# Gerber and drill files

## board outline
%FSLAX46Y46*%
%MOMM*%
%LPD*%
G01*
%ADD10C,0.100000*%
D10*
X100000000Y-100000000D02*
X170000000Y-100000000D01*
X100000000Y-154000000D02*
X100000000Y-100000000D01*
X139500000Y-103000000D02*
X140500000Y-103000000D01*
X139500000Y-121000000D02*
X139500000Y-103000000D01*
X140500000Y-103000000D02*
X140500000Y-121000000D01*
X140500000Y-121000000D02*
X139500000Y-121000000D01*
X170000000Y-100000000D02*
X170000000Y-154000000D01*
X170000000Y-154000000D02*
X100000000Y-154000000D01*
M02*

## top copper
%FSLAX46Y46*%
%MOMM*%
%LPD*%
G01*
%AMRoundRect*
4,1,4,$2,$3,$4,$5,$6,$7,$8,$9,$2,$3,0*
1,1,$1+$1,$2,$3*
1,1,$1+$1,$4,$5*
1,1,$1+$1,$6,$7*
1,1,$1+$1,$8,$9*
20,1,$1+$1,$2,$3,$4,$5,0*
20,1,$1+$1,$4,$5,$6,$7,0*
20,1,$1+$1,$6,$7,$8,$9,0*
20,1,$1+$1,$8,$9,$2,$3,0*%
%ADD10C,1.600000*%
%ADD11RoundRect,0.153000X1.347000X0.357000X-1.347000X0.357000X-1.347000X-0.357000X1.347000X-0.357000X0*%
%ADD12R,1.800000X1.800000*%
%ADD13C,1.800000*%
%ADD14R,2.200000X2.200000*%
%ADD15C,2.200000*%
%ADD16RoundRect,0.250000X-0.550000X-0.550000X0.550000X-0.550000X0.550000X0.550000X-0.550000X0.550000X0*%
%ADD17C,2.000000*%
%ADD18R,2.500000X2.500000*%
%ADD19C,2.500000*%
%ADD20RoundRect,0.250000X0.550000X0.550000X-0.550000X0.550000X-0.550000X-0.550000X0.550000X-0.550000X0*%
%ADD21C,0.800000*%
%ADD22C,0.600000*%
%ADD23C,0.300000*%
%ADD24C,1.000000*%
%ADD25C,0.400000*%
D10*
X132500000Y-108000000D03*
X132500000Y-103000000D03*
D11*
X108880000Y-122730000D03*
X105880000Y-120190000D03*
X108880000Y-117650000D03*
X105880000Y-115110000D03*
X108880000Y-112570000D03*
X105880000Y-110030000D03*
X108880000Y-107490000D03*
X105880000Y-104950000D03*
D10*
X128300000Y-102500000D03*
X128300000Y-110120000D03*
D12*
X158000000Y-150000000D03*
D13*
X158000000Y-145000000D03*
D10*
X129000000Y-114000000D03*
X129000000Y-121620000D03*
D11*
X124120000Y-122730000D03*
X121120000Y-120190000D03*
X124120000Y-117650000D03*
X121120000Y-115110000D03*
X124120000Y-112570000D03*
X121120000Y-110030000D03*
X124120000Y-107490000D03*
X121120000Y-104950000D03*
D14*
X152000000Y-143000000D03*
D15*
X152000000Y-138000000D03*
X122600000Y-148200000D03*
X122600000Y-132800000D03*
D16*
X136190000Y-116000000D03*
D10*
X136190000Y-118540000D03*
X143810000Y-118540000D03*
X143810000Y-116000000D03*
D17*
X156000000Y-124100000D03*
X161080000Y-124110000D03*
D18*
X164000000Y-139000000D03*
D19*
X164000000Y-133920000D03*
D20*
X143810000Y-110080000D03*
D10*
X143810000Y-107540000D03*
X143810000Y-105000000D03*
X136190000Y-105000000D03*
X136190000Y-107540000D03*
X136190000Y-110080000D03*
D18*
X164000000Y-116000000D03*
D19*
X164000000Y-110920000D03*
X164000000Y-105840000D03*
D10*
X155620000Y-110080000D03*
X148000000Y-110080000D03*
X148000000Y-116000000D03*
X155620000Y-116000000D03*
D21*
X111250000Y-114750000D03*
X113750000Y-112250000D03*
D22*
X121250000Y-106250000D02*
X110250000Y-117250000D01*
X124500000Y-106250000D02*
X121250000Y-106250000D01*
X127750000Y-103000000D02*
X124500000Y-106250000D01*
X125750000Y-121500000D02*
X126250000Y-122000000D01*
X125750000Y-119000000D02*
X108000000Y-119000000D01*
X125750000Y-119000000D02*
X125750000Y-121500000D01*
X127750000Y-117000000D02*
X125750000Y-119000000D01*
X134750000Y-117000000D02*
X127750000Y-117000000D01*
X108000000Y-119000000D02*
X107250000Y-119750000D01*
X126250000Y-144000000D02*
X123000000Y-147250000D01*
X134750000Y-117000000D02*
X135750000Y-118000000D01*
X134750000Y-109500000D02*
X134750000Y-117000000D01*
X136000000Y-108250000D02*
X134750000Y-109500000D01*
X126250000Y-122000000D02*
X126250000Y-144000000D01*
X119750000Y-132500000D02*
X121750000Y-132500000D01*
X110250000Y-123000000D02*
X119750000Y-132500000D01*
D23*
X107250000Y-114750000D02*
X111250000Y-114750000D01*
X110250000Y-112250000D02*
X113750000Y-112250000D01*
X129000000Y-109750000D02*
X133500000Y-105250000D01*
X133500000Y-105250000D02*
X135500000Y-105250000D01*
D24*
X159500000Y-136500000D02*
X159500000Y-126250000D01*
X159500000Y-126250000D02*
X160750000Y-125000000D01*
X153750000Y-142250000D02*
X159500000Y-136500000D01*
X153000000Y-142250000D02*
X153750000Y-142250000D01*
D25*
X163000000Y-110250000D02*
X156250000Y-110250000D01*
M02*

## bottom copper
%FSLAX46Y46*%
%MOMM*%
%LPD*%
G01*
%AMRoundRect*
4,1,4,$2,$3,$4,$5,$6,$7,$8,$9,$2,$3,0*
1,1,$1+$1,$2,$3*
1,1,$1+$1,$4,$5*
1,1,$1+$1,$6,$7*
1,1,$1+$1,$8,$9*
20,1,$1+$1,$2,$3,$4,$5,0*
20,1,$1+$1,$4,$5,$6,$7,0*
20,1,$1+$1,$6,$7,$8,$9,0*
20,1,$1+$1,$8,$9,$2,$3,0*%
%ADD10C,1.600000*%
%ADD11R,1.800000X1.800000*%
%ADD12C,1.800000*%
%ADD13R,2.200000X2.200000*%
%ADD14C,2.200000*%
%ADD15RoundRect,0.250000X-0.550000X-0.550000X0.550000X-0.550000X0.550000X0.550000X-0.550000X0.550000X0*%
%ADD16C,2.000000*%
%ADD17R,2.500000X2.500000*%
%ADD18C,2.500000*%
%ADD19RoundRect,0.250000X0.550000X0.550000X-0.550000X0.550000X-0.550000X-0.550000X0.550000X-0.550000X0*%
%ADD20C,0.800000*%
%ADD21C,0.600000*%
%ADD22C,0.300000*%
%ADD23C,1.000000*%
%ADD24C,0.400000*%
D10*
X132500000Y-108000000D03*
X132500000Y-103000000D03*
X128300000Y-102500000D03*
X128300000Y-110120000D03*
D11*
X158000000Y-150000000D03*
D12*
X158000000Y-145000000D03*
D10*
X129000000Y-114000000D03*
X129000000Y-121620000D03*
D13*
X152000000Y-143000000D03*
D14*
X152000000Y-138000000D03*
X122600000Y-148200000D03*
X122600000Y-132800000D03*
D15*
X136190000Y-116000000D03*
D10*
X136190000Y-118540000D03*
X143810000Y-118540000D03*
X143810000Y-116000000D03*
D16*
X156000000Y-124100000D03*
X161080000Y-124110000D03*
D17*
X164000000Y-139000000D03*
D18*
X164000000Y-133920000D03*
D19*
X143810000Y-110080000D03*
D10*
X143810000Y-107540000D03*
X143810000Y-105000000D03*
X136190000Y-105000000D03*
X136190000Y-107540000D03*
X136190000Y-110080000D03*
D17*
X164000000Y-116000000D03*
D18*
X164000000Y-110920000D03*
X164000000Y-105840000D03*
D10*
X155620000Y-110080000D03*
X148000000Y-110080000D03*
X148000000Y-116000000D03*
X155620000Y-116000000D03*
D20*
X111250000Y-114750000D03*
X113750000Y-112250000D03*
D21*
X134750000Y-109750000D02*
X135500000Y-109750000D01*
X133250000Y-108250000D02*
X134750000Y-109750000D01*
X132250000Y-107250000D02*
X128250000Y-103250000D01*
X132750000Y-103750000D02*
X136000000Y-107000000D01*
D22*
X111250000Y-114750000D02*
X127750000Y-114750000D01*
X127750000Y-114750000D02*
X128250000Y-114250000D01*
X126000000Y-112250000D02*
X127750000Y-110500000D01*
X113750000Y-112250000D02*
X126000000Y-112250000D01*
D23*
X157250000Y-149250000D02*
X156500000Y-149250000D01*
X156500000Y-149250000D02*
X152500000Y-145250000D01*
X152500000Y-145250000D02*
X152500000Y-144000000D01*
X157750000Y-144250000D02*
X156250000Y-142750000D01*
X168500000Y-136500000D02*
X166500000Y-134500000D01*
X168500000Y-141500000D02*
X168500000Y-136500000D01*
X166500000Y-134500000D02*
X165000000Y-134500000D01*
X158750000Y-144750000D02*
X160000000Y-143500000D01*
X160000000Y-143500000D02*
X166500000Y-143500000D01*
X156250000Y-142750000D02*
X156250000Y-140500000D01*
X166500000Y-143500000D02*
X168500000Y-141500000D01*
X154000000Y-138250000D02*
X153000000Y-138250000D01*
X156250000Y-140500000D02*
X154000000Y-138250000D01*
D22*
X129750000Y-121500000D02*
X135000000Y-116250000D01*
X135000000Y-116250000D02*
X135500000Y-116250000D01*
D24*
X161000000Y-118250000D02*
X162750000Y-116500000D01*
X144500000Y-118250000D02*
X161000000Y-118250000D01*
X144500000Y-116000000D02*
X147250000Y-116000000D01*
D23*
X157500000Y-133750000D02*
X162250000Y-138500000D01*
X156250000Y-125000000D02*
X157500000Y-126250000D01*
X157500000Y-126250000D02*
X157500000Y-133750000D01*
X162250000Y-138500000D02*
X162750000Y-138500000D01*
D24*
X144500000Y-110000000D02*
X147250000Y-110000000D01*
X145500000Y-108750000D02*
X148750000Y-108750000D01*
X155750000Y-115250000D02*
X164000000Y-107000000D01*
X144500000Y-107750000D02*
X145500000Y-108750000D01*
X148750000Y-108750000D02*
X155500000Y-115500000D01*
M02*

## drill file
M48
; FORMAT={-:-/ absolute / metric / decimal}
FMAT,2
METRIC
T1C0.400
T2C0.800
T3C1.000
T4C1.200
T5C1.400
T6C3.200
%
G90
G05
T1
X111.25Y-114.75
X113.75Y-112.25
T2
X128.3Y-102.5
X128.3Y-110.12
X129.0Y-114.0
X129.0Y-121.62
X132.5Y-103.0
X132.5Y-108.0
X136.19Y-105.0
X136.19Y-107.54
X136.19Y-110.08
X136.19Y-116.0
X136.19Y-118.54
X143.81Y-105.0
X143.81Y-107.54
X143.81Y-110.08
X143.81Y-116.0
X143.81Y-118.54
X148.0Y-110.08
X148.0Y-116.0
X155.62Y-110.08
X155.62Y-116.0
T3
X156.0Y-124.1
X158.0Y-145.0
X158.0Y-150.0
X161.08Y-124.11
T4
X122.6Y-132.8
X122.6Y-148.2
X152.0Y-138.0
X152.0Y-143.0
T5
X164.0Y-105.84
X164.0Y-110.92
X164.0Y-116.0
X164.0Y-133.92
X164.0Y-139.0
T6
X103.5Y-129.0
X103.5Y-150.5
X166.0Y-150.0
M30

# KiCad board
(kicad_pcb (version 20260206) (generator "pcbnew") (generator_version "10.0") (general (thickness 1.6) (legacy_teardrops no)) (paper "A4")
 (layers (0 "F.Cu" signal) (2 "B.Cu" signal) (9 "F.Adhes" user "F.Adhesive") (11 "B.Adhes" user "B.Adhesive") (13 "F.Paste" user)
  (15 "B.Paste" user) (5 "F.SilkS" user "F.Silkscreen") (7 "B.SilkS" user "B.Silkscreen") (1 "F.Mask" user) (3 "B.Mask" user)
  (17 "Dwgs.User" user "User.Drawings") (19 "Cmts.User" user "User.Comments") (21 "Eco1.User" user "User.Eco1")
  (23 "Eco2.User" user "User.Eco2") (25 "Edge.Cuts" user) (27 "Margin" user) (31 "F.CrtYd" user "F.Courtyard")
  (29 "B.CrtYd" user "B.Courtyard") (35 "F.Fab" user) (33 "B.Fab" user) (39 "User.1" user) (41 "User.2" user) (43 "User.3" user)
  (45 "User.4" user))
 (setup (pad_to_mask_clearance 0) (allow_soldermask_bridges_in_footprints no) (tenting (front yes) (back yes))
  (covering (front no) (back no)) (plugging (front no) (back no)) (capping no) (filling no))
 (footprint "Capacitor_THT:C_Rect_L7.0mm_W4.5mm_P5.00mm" (layer "F.Cu") (at 132.5 108 90)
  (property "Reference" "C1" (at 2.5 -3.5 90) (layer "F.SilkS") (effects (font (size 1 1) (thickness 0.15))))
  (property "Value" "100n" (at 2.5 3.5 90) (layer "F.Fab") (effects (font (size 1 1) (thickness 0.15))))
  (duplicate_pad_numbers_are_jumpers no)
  (pad "1" thru_hole circle (at 0 0 90) (size 1.6 1.6) (drill 0.8) (layers "*.Cu" "*.Mask") (remove_unused_layers no) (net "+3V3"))
  (pad "2" thru_hole circle (at 5 0 90) (size 1.6 1.6) (drill 0.8) (layers "*.Cu" "*.Mask") (remove_unused_layers no) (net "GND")))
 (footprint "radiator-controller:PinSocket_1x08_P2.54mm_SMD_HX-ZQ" (layer "F.Cu") (at 107.38 113.84 180)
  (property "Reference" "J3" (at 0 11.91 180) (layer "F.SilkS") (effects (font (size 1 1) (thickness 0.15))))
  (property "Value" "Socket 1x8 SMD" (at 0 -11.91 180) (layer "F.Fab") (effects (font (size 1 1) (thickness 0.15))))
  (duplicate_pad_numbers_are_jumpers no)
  (pad "1" smd roundrect (at -1.5 -8.89 180) (size 3 1.02) (layers "F.Cu" "F.Mask" "F.Paste") (roundrect_rratio 0.15) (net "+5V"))
  (pad "2" smd roundrect (at 1.5 -6.35 180) (size 3 1.02) (layers "F.Cu" "F.Mask" "F.Paste") (roundrect_rratio 0.15) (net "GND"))
  (pad "3" smd roundrect (at -1.5 -3.81 180) (size 3 1.02) (layers "F.Cu" "F.Mask" "F.Paste") (roundrect_rratio 0.15) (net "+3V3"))
  (pad "4" smd roundrect (at 1.5 -1.27 180) (size 3 1.02) (layers "F.Cu" "F.Mask" "F.Paste") (roundrect_rratio 0.15) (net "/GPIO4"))
  (pad "5" smd roundrect (at -1.5 1.27 180) (size 3 1.02) (layers "F.Cu" "F.Mask" "F.Paste") (roundrect_rratio 0.15) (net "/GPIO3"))
  (pad "6" smd roundrect (at 1.5 3.81 180) (size 3 1.02) (layers "F.Cu" "F.Mask" "F.Paste") (roundrect_rratio 0.15) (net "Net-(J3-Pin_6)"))
  (pad "7" smd roundrect (at -1.5 6.35 180) (size 3 1.02) (layers "F.Cu" "F.Mask" "F.Paste") (roundrect_rratio 0.15) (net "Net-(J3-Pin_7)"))
  (pad "8" smd roundrect (at 1.5 8.89 180) (size 3 1.02) (layers "F.Cu" "F.Mask" "F.Paste") (roundrect_rratio 0.15) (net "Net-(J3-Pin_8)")))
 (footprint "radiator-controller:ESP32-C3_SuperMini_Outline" (layer "F.Cu") (at 115 113 180)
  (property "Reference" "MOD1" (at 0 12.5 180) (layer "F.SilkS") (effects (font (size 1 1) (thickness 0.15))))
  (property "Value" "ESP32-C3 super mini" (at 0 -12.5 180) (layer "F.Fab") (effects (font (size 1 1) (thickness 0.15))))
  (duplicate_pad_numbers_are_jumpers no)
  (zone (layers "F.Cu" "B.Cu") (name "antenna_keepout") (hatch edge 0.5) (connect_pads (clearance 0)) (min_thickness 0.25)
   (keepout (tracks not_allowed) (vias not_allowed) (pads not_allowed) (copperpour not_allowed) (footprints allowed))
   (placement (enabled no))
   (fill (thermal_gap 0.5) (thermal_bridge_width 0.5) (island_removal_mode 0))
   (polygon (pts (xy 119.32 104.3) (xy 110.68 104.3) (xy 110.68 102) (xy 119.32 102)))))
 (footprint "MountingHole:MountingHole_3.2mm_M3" (layer "F.Cu") (at 166 150)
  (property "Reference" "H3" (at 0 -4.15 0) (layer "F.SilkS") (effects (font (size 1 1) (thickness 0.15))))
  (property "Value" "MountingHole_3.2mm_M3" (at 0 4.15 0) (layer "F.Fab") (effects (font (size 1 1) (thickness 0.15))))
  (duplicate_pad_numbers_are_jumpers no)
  (pad "" np_thru_hole circle (at 0 0) (size 3.2 3.2) (drill 3.2) (layers "*.Cu" "*.Mask")))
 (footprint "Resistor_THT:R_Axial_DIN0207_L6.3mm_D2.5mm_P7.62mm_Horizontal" (layer "F.Cu") (at 128.3 102.5 -90)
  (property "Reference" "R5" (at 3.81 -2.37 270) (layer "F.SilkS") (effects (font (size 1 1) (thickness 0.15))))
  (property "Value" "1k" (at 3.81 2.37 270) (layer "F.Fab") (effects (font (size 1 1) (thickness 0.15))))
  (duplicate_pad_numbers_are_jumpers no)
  (pad "1" thru_hole circle (at 0 0 270) (size 1.6 1.6) (drill 0.8) (layers "*.Cu" "*.Mask") (remove_unused_layers no) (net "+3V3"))
  (pad "2" thru_hole circle (at 7.62 0 270) (size 1.6 1.6) (drill 0.8) (layers "*.Cu" "*.Mask") (remove_unused_layers no) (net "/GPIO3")))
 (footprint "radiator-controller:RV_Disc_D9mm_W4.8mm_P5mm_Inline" (layer "F.Cu") (at 158 150 90)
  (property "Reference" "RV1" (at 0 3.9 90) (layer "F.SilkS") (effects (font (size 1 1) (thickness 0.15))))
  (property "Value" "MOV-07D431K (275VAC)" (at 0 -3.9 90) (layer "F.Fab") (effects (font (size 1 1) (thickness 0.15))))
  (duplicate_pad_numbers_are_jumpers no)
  (pad "1" thru_hole rect (at 0 0 90) (size 1.8 1.8) (drill 1) (layers "*.Cu" "*.Mask") (remove_unused_layers no) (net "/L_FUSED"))
  (pad "2" thru_hole circle (at 5 0 90) (size 1.8 1.8) (drill 1) (layers "*.Cu" "*.Mask") (remove_unused_layers no) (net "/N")))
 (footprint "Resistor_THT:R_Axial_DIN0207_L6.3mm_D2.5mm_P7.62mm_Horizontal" (layer "F.Cu") (at 129 114 -90)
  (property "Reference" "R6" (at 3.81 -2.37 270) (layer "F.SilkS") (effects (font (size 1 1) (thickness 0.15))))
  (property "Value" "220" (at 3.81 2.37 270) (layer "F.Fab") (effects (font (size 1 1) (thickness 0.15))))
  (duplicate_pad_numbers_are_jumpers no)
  (pad "1" thru_hole circle (at 0 0 270) (size 1.6 1.6) (drill 0.8) (layers "*.Cu" "*.Mask") (remove_unused_layers no) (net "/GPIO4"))
  (pad "2" thru_hole circle (at 7.62 0 270) (size 1.6 1.6) (drill 0.8) (layers "*.Cu" "*.Mask") (remove_unused_layers no)
   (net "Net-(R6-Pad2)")))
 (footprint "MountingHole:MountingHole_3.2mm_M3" (layer "F.Cu") (at 103.5 129)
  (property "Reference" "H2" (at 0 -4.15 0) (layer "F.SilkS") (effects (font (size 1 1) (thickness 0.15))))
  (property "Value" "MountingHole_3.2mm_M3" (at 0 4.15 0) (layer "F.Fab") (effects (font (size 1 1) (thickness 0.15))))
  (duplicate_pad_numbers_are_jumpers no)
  (pad "" np_thru_hole circle (at 0 0) (size 3.2 3.2) (drill 3.2) (layers "*.Cu" "*.Mask")))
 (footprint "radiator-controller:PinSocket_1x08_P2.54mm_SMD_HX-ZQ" (layer "F.Cu") (at 122.62 113.84 180)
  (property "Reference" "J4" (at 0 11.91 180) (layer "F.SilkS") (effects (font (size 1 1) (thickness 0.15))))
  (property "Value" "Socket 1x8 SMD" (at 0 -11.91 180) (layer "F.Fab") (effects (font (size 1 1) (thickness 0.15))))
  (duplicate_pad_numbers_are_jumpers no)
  (pad "1" smd roundrect (at -1.5 -8.89 180) (size 3 1.02) (layers "F.Cu" "F.Mask" "F.Paste") (roundrect_rratio 0.15) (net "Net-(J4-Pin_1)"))
  (pad "2" smd roundrect (at 1.5 -6.35 180) (size 3 1.02) (layers "F.Cu" "F.Mask" "F.Paste") (roundrect_rratio 0.15) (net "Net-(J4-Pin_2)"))
  (pad "3" smd roundrect (at -1.5 -3.81 180) (size 3 1.02) (layers "F.Cu" "F.Mask" "F.Paste") (roundrect_rratio 0.15) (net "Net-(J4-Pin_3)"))
  (pad "4" smd roundrect (at 1.5 -1.27 180) (size 3 1.02) (layers "F.Cu" "F.Mask" "F.Paste") (roundrect_rratio 0.15) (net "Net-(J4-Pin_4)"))
  (pad "5" smd roundrect (at -1.5 1.27 180) (size 3 1.02) (layers "F.Cu" "F.Mask" "F.Paste") (roundrect_rratio 0.15) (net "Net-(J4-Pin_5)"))
  (pad "6" smd roundrect (at 1.5 3.81 180) (size 3 1.02) (layers "F.Cu" "F.Mask" "F.Paste") (roundrect_rratio 0.15) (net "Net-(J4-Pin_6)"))
  (pad "7" smd roundrect (at -1.5 6.35 180) (size 3 1.02) (layers "F.Cu" "F.Mask" "F.Paste") (roundrect_rratio 0.15) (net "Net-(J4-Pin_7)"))
  (pad "8" smd roundrect (at 1.5 8.89 180) (size 3 1.02) (layers "F.Cu" "F.Mask" "F.Paste") (roundrect_rratio 0.15) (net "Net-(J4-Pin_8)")))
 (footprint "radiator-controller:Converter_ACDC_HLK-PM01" (layer "F.Cu") (at 152 143 180)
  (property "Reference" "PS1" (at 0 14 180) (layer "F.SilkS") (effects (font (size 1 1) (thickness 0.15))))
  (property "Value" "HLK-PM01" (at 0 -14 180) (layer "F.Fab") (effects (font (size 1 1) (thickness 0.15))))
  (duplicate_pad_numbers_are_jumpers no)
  (pad "1" thru_hole rect (at 0 0 180) (size 2.2 2.2) (drill 1.2) (layers "*.Cu" "*.Mask") (remove_unused_layers no) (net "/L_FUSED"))
  (pad "2" thru_hole circle (at 0 5 180) (size 2.2 2.2) (drill 1.2) (layers "*.Cu" "*.Mask") (remove_unused_layers no) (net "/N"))
  (pad "3" thru_hole circle (at 29.4 -5.2 180) (size 2.2 2.2) (drill 1.2) (layers "*.Cu" "*.Mask") (remove_unused_layers no) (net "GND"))
  (pad "4" thru_hole circle (at 29.4 10.2 180) (size 2.2 2.2) (drill 1.2) (layers "*.Cu" "*.Mask") (remove_unused_layers no) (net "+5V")))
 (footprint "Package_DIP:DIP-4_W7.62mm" (layer "F.Cu") (at 136.19 116)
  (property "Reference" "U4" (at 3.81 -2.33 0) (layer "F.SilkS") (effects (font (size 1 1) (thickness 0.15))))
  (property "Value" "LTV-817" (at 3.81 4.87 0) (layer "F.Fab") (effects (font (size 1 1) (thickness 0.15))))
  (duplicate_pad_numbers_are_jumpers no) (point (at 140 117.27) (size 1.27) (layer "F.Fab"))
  (pad "1" thru_hole roundrect (at 0 0) (size 1.6 1.6) (drill 0.8) (layers "*.Cu" "*.Mask") (remove_unused_layers no)
   (roundrect_rratio 0.15625) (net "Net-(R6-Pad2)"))
  (pad "2" thru_hole circle (at 0 2.54) (size 1.6 1.6) (drill 0.8) (layers "*.Cu" "*.Mask") (remove_unused_layers no) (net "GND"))
  (pad "3" thru_hole circle (at 7.62 2.54) (size 1.6 1.6) (drill 0.8) (layers "*.Cu" "*.Mask") (remove_unused_layers no) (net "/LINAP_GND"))
  (pad "4" thru_hole circle (at 7.62 0) (size 1.6 1.6) (drill 0.8) (layers "*.Cu" "*.Mask") (remove_unused_layers no) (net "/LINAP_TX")))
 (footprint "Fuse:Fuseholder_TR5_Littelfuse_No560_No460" (layer "F.Cu") (at 156 124.1)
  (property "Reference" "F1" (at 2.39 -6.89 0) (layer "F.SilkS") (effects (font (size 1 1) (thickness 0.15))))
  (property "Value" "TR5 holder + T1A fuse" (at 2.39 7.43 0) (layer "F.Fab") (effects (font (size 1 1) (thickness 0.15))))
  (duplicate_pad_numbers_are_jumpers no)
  (pad "1" thru_hole circle (at 0 0) (size 2 2) (drill 1) (layers "*.Cu" "*.Mask") (remove_unused_layers no) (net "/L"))
  (pad "2" thru_hole circle (at 5.08 0.01) (size 2 2) (drill 1) (layers "*.Cu" "*.Mask") (remove_unused_layers no) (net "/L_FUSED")))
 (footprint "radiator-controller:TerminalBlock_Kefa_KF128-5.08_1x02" (layer "F.Cu") (at 164 139 90)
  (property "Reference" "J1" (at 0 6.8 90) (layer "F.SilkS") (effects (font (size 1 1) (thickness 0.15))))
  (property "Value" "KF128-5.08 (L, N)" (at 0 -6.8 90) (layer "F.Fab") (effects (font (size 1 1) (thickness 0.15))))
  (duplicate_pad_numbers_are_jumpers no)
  (pad "1" thru_hole rect (at 0 0 90) (size 2.5 2.5) (drill 1.4) (layers "*.Cu" "*.Mask") (remove_unused_layers no) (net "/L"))
  (pad "2" thru_hole circle (at 5.08 0 90) (size 2.5 2.5) (drill 1.4) (layers "*.Cu" "*.Mask") (remove_unused_layers no) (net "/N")))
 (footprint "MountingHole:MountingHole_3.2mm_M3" (layer "F.Cu") (at 103.5 150.5)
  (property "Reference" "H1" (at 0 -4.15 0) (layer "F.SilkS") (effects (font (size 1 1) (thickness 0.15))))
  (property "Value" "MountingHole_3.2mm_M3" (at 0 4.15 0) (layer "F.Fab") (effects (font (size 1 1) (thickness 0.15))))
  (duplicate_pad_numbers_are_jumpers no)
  (pad "" np_thru_hole circle (at 0 0) (size 3.2 3.2) (drill 3.2) (layers "*.Cu" "*.Mask")))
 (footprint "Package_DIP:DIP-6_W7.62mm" (layer "F.Cu") (at 143.81 110.08 180)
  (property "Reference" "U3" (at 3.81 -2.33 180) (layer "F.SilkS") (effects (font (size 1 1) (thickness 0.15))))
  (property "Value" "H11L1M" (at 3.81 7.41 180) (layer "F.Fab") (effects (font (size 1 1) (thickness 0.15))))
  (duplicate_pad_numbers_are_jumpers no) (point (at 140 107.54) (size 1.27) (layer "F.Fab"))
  (pad "1" thru_hole roundrect (at 0 0 180) (size 1.6 1.6) (drill 0.8) (layers "*.Cu" "*.Mask") (remove_unused_layers no)
   (roundrect_rratio 0.15625) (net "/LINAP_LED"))
  (pad "2" thru_hole circle (at 0 2.54 180) (size 1.6 1.6) (drill 0.8) (layers "*.Cu" "*.Mask") (remove_unused_layers no)
   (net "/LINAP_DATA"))
  (pad "3" thru_hole circle (at 0 5.08 180) (size 1.6 1.6) (drill 0.8) (layers "*.Cu" "*.Mask") (remove_unused_layers no)
   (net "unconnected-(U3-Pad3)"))
  (pad "4" thru_hole circle (at 7.62 5.08 180) (size 1.6 1.6) (drill 0.8) (layers "*.Cu" "*.Mask") (remove_unused_layers no) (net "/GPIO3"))
  (pad "5" thru_hole circle (at 7.62 2.54 180) (size 1.6 1.6) (drill 0.8) (layers "*.Cu" "*.Mask") (remove_unused_layers no) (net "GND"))
  (pad "6" thru_hole circle (at 7.62 0 180) (size 1.6 1.6) (drill 0.8) (layers "*.Cu" "*.Mask") (remove_unused_layers no) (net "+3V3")))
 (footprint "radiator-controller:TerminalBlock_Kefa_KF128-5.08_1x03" (layer "F.Cu") (at 164 116 90)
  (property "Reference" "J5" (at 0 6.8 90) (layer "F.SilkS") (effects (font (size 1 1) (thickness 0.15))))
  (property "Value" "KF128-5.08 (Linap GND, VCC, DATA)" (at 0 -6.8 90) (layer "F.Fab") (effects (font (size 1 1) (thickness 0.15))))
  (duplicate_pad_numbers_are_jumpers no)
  (pad "1" thru_hole rect (at 0 0 90) (size 2.5 2.5) (drill 1.4) (layers "*.Cu" "*.Mask") (remove_unused_layers no) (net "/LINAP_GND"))
  (pad "2" thru_hole circle (at 5.08 0 90) (size 2.5 2.5) (drill 1.4) (layers "*.Cu" "*.Mask") (remove_unused_layers no) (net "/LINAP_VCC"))
  (pad "3" thru_hole circle (at 10.16 0 90) (size 2.5 2.5) (drill 1.4) (layers "*.Cu" "*.Mask") (remove_unused_layers no)
   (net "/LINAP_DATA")))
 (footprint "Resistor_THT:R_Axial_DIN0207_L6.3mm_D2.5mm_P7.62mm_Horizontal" (layer "F.Cu") (at 155.62 110.08 180)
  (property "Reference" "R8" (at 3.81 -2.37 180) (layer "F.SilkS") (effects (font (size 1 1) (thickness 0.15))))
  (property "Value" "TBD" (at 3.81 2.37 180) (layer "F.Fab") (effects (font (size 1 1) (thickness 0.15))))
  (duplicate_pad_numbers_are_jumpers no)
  (pad "1" thru_hole circle (at 0 0 180) (size 1.6 1.6) (drill 0.8) (layers "*.Cu" "*.Mask") (remove_unused_layers no) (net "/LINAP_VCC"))
  (pad "2" thru_hole circle (at 7.62 0 180) (size 1.6 1.6) (drill 0.8) (layers "*.Cu" "*.Mask") (remove_unused_layers no) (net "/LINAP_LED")))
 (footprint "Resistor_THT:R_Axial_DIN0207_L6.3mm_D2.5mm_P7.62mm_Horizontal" (layer "F.Cu") (at 148 116)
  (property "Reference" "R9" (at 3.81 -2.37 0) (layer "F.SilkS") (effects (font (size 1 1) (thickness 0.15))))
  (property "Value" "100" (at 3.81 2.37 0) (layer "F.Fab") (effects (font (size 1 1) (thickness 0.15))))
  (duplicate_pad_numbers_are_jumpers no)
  (pad "1" thru_hole circle (at 0 0) (size 1.6 1.6) (drill 0.8) (layers "*.Cu" "*.Mask") (remove_unused_layers no) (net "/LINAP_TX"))
  (pad "2" thru_hole circle (at 7.62 0) (size 1.6 1.6) (drill 0.8) (layers "*.Cu" "*.Mask") (remove_unused_layers no) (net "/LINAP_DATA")))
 (gr_line (start 100 100) (end 170 100) (stroke (width 0.1) (type default)) (layer "Edge.Cuts"))
 (gr_line (start 100 154) (end 100 100) (stroke (width 0.1) (type default)) (layer "Edge.Cuts"))
 (gr_line (start 139.5 103) (end 140.5 103) (stroke (width 0.1) (type default)) (layer "Edge.Cuts"))
 (gr_line (start 139.5 121) (end 139.5 103) (stroke (width 0.1) (type default)) (layer "Edge.Cuts"))
 (gr_line (start 140.5 103) (end 140.5 121) (stroke (width 0.1) (type default)) (layer "Edge.Cuts"))
 (gr_line (start 140.5 121) (end 139.5 121) (stroke (width 0.1) (type default)) (layer "Edge.Cuts"))
 (gr_line (start 170 100) (end 170 154) (stroke (width 0.1) (type default)) (layer "Edge.Cuts"))
 (gr_line (start 170 154) (end 100 154) (stroke (width 0.1) (type default)) (layer "Edge.Cuts"))
 (segment (start 121.25 106.25) (end 110.25 117.25) (width 0.6) (layer "F.Cu") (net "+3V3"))
 (segment (start 124.5 106.25) (end 121.25 106.25) (width 0.6) (layer "F.Cu") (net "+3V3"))
 (segment (start 127.75 103) (end 124.5 106.25) (width 0.6) (layer "F.Cu") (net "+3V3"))
 (segment (start 134.75 109.75) (end 135.5 109.75) (width 0.6) (layer "B.Cu") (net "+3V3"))
 (segment (start 133.25 108.25) (end 134.75 109.75) (width 0.6) (layer "B.Cu") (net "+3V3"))
 (segment (start 132.25 107.25) (end 128.25 103.25) (width 0.6) (layer "B.Cu") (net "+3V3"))
 (segment (start 125.75 121.5) (end 126.25 122) (width 0.6) (layer "F.Cu") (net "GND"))
 (segment (start 125.75 119) (end 108 119) (width 0.6) (layer "F.Cu") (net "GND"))
 (segment (start 125.75 119) (end 125.75 121.5) (width 0.6) (layer "F.Cu") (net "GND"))
 (segment (start 127.75 117) (end 125.75 119) (width 0.6) (layer "F.Cu") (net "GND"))
 (segment (start 134.75 117) (end 127.75 117) (width 0.6) (layer "F.Cu") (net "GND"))
 (segment (start 108 119) (end 107.25 119.75) (width 0.6) (layer "F.Cu") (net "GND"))
 (segment (start 126.25 144) (end 123 147.25) (width 0.6) (layer "F.Cu") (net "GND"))
 (segment (start 134.75 117) (end 135.75 118) (width 0.6) (layer "F.Cu") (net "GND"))
 (segment (start 134.75 109.5) (end 134.75 117) (width 0.6) (layer "F.Cu") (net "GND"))
 (segment (start 136 108.25) (end 134.75 109.5) (width 0.6) (layer "F.Cu") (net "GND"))
 (segment (start 126.25 122) (end 126.25 144) (width 0.6) (layer "F.Cu") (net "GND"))
 (segment (start 132.75 103.75) (end 136 107) (width 0.6) (layer "B.Cu") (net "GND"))
 (segment (start 119.75 132.5) (end 121.75 132.5) (width 0.6) (layer "F.Cu") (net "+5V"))
 (segment (start 110.25 123) (end 119.75 132.5) (width 0.6) (layer "F.Cu") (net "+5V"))
 (segment (start 107.25 114.75) (end 111.25 114.75) (width 0.3) (layer "F.Cu") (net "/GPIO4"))
 (via (at 111.25 114.75) (size 0.8) (drill 0.4) (layers "F.Cu" "B.Cu") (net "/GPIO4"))
 (segment (start 111.25 114.75) (end 127.75 114.75) (width 0.3) (layer "B.Cu") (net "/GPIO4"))
 (segment (start 127.75 114.75) (end 128.25 114.25) (width 0.3) (layer "B.Cu") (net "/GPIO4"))
 (segment (start 110.25 112.25) (end 113.75 112.25) (width 0.3) (layer "F.Cu") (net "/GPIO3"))
 (segment (start 129 109.75) (end 133.5 105.25) (width 0.3) (layer "F.Cu") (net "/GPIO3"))
 (segment (start 133.5 105.25) (end 135.5 105.25) (width 0.3) (layer "F.Cu") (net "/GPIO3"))
 (via (at 113.75 112.25) (size 0.8) (drill 0.4) (layers "F.Cu" "B.Cu") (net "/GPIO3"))
 (segment (start 126 112.25) (end 127.75 110.5) (width 0.3) (layer "B.Cu") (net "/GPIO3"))
 (segment (start 113.75 112.25) (end 126 112.25) (width 0.3) (layer "B.Cu") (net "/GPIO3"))
 (segment (start 159.5 136.5) (end 159.5 126.25) (width 1) (layer "F.Cu") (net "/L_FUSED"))
 (segment (start 159.5 126.25) (end 160.75 125) (width 1) (layer "F.Cu") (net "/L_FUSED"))
 (segment (start 153.75 142.25) (end 159.5 136.5) (width 1) (layer "F.Cu") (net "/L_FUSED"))
 (segment (start 153 142.25) (end 153.75 142.25) (width 1) (layer "F.Cu") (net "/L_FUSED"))
 (segment (start 157.25 149.25) (end 156.5 149.25) (width 1) (layer "B.Cu") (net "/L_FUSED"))
 (segment (start 156.5 149.25) (end 152.5 145.25) (width 1) (layer "B.Cu") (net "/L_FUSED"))
 (segment (start 152.5 145.25) (end 152.5 144) (width 1) (layer "B.Cu") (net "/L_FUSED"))
 (segment (start 157.75 144.25) (end 156.25 142.75) (width 1) (layer "B.Cu") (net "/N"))
 (segment (start 168.5 136.5) (end 166.5 134.5) (width 1) (layer "B.Cu") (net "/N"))
 (segment (start 168.5 141.5) (end 168.5 136.5) (width 1) (layer "B.Cu") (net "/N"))
 (segment (start 166.5 134.5) (end 165 134.5) (width 1) (layer "B.Cu") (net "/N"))
 (segment (start 158.75 144.75) (end 160 143.5) (width 1) (layer "B.Cu") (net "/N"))
 (segment (start 160 143.5) (end 166.5 143.5) (width 1) (layer "B.Cu") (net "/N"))
 (segment (start 156.25 142.75) (end 156.25 140.5) (width 1) (layer "B.Cu") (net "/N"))
 (segment (start 166.5 143.5) (end 168.5 141.5) (width 1) (layer "B.Cu") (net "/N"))
 (segment (start 154 138.25) (end 153 138.25) (width 1) (layer "B.Cu") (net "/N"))
 (segment (start 156.25 140.5) (end 154 138.25) (width 1) (layer "B.Cu") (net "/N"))
 (segment (start 129.75 121.5) (end 135 116.25) (width 0.3) (layer "B.Cu") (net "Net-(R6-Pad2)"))
 (segment (start 135 116.25) (end 135.5 116.25) (width 0.3) (layer "B.Cu") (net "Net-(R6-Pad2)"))
 (segment (start 161 118.25) (end 162.75 116.5) (width 0.4) (layer "B.Cu") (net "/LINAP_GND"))
 (segment (start 144.5 118.25) (end 161 118.25) (width 0.4) (layer "B.Cu") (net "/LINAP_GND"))
 (segment (start 144.5 116) (end 147.25 116) (width 0.4) (layer "B.Cu") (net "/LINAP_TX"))
 (segment (start 157.5 133.75) (end 162.25 138.5) (width 1) (layer "B.Cu") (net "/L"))
 (segment (start 156.25 125) (end 157.5 126.25) (width 1) (layer "B.Cu") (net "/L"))
 (segment (start 157.5 126.25) (end 157.5 133.75) (width 1) (layer "B.Cu") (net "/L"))
 (segment (start 162.25 138.5) (end 162.75 138.5) (width 1) (layer "B.Cu") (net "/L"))
 (segment (start 144.5 110) (end 147.25 110) (width 0.4) (layer "B.Cu") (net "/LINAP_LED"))
 (segment (start 145.5 108.75) (end 148.75 108.75) (width 0.4) (layer "B.Cu") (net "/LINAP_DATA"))
 (segment (start 155.75 115.25) (end 164 107) (width 0.4) (layer "B.Cu") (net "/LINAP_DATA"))
 (segment (start 144.5 107.75) (end 145.5 108.75) (width 0.4) (layer "B.Cu") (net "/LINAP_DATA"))
 (segment (start 148.75 108.75) (end 155.5 115.5) (width 0.4) (layer "B.Cu") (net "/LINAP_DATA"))
 (segment (start 163 110.25) (end 156.25 110.25) (width 0.4) (layer "F.Cu") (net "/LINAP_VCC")))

